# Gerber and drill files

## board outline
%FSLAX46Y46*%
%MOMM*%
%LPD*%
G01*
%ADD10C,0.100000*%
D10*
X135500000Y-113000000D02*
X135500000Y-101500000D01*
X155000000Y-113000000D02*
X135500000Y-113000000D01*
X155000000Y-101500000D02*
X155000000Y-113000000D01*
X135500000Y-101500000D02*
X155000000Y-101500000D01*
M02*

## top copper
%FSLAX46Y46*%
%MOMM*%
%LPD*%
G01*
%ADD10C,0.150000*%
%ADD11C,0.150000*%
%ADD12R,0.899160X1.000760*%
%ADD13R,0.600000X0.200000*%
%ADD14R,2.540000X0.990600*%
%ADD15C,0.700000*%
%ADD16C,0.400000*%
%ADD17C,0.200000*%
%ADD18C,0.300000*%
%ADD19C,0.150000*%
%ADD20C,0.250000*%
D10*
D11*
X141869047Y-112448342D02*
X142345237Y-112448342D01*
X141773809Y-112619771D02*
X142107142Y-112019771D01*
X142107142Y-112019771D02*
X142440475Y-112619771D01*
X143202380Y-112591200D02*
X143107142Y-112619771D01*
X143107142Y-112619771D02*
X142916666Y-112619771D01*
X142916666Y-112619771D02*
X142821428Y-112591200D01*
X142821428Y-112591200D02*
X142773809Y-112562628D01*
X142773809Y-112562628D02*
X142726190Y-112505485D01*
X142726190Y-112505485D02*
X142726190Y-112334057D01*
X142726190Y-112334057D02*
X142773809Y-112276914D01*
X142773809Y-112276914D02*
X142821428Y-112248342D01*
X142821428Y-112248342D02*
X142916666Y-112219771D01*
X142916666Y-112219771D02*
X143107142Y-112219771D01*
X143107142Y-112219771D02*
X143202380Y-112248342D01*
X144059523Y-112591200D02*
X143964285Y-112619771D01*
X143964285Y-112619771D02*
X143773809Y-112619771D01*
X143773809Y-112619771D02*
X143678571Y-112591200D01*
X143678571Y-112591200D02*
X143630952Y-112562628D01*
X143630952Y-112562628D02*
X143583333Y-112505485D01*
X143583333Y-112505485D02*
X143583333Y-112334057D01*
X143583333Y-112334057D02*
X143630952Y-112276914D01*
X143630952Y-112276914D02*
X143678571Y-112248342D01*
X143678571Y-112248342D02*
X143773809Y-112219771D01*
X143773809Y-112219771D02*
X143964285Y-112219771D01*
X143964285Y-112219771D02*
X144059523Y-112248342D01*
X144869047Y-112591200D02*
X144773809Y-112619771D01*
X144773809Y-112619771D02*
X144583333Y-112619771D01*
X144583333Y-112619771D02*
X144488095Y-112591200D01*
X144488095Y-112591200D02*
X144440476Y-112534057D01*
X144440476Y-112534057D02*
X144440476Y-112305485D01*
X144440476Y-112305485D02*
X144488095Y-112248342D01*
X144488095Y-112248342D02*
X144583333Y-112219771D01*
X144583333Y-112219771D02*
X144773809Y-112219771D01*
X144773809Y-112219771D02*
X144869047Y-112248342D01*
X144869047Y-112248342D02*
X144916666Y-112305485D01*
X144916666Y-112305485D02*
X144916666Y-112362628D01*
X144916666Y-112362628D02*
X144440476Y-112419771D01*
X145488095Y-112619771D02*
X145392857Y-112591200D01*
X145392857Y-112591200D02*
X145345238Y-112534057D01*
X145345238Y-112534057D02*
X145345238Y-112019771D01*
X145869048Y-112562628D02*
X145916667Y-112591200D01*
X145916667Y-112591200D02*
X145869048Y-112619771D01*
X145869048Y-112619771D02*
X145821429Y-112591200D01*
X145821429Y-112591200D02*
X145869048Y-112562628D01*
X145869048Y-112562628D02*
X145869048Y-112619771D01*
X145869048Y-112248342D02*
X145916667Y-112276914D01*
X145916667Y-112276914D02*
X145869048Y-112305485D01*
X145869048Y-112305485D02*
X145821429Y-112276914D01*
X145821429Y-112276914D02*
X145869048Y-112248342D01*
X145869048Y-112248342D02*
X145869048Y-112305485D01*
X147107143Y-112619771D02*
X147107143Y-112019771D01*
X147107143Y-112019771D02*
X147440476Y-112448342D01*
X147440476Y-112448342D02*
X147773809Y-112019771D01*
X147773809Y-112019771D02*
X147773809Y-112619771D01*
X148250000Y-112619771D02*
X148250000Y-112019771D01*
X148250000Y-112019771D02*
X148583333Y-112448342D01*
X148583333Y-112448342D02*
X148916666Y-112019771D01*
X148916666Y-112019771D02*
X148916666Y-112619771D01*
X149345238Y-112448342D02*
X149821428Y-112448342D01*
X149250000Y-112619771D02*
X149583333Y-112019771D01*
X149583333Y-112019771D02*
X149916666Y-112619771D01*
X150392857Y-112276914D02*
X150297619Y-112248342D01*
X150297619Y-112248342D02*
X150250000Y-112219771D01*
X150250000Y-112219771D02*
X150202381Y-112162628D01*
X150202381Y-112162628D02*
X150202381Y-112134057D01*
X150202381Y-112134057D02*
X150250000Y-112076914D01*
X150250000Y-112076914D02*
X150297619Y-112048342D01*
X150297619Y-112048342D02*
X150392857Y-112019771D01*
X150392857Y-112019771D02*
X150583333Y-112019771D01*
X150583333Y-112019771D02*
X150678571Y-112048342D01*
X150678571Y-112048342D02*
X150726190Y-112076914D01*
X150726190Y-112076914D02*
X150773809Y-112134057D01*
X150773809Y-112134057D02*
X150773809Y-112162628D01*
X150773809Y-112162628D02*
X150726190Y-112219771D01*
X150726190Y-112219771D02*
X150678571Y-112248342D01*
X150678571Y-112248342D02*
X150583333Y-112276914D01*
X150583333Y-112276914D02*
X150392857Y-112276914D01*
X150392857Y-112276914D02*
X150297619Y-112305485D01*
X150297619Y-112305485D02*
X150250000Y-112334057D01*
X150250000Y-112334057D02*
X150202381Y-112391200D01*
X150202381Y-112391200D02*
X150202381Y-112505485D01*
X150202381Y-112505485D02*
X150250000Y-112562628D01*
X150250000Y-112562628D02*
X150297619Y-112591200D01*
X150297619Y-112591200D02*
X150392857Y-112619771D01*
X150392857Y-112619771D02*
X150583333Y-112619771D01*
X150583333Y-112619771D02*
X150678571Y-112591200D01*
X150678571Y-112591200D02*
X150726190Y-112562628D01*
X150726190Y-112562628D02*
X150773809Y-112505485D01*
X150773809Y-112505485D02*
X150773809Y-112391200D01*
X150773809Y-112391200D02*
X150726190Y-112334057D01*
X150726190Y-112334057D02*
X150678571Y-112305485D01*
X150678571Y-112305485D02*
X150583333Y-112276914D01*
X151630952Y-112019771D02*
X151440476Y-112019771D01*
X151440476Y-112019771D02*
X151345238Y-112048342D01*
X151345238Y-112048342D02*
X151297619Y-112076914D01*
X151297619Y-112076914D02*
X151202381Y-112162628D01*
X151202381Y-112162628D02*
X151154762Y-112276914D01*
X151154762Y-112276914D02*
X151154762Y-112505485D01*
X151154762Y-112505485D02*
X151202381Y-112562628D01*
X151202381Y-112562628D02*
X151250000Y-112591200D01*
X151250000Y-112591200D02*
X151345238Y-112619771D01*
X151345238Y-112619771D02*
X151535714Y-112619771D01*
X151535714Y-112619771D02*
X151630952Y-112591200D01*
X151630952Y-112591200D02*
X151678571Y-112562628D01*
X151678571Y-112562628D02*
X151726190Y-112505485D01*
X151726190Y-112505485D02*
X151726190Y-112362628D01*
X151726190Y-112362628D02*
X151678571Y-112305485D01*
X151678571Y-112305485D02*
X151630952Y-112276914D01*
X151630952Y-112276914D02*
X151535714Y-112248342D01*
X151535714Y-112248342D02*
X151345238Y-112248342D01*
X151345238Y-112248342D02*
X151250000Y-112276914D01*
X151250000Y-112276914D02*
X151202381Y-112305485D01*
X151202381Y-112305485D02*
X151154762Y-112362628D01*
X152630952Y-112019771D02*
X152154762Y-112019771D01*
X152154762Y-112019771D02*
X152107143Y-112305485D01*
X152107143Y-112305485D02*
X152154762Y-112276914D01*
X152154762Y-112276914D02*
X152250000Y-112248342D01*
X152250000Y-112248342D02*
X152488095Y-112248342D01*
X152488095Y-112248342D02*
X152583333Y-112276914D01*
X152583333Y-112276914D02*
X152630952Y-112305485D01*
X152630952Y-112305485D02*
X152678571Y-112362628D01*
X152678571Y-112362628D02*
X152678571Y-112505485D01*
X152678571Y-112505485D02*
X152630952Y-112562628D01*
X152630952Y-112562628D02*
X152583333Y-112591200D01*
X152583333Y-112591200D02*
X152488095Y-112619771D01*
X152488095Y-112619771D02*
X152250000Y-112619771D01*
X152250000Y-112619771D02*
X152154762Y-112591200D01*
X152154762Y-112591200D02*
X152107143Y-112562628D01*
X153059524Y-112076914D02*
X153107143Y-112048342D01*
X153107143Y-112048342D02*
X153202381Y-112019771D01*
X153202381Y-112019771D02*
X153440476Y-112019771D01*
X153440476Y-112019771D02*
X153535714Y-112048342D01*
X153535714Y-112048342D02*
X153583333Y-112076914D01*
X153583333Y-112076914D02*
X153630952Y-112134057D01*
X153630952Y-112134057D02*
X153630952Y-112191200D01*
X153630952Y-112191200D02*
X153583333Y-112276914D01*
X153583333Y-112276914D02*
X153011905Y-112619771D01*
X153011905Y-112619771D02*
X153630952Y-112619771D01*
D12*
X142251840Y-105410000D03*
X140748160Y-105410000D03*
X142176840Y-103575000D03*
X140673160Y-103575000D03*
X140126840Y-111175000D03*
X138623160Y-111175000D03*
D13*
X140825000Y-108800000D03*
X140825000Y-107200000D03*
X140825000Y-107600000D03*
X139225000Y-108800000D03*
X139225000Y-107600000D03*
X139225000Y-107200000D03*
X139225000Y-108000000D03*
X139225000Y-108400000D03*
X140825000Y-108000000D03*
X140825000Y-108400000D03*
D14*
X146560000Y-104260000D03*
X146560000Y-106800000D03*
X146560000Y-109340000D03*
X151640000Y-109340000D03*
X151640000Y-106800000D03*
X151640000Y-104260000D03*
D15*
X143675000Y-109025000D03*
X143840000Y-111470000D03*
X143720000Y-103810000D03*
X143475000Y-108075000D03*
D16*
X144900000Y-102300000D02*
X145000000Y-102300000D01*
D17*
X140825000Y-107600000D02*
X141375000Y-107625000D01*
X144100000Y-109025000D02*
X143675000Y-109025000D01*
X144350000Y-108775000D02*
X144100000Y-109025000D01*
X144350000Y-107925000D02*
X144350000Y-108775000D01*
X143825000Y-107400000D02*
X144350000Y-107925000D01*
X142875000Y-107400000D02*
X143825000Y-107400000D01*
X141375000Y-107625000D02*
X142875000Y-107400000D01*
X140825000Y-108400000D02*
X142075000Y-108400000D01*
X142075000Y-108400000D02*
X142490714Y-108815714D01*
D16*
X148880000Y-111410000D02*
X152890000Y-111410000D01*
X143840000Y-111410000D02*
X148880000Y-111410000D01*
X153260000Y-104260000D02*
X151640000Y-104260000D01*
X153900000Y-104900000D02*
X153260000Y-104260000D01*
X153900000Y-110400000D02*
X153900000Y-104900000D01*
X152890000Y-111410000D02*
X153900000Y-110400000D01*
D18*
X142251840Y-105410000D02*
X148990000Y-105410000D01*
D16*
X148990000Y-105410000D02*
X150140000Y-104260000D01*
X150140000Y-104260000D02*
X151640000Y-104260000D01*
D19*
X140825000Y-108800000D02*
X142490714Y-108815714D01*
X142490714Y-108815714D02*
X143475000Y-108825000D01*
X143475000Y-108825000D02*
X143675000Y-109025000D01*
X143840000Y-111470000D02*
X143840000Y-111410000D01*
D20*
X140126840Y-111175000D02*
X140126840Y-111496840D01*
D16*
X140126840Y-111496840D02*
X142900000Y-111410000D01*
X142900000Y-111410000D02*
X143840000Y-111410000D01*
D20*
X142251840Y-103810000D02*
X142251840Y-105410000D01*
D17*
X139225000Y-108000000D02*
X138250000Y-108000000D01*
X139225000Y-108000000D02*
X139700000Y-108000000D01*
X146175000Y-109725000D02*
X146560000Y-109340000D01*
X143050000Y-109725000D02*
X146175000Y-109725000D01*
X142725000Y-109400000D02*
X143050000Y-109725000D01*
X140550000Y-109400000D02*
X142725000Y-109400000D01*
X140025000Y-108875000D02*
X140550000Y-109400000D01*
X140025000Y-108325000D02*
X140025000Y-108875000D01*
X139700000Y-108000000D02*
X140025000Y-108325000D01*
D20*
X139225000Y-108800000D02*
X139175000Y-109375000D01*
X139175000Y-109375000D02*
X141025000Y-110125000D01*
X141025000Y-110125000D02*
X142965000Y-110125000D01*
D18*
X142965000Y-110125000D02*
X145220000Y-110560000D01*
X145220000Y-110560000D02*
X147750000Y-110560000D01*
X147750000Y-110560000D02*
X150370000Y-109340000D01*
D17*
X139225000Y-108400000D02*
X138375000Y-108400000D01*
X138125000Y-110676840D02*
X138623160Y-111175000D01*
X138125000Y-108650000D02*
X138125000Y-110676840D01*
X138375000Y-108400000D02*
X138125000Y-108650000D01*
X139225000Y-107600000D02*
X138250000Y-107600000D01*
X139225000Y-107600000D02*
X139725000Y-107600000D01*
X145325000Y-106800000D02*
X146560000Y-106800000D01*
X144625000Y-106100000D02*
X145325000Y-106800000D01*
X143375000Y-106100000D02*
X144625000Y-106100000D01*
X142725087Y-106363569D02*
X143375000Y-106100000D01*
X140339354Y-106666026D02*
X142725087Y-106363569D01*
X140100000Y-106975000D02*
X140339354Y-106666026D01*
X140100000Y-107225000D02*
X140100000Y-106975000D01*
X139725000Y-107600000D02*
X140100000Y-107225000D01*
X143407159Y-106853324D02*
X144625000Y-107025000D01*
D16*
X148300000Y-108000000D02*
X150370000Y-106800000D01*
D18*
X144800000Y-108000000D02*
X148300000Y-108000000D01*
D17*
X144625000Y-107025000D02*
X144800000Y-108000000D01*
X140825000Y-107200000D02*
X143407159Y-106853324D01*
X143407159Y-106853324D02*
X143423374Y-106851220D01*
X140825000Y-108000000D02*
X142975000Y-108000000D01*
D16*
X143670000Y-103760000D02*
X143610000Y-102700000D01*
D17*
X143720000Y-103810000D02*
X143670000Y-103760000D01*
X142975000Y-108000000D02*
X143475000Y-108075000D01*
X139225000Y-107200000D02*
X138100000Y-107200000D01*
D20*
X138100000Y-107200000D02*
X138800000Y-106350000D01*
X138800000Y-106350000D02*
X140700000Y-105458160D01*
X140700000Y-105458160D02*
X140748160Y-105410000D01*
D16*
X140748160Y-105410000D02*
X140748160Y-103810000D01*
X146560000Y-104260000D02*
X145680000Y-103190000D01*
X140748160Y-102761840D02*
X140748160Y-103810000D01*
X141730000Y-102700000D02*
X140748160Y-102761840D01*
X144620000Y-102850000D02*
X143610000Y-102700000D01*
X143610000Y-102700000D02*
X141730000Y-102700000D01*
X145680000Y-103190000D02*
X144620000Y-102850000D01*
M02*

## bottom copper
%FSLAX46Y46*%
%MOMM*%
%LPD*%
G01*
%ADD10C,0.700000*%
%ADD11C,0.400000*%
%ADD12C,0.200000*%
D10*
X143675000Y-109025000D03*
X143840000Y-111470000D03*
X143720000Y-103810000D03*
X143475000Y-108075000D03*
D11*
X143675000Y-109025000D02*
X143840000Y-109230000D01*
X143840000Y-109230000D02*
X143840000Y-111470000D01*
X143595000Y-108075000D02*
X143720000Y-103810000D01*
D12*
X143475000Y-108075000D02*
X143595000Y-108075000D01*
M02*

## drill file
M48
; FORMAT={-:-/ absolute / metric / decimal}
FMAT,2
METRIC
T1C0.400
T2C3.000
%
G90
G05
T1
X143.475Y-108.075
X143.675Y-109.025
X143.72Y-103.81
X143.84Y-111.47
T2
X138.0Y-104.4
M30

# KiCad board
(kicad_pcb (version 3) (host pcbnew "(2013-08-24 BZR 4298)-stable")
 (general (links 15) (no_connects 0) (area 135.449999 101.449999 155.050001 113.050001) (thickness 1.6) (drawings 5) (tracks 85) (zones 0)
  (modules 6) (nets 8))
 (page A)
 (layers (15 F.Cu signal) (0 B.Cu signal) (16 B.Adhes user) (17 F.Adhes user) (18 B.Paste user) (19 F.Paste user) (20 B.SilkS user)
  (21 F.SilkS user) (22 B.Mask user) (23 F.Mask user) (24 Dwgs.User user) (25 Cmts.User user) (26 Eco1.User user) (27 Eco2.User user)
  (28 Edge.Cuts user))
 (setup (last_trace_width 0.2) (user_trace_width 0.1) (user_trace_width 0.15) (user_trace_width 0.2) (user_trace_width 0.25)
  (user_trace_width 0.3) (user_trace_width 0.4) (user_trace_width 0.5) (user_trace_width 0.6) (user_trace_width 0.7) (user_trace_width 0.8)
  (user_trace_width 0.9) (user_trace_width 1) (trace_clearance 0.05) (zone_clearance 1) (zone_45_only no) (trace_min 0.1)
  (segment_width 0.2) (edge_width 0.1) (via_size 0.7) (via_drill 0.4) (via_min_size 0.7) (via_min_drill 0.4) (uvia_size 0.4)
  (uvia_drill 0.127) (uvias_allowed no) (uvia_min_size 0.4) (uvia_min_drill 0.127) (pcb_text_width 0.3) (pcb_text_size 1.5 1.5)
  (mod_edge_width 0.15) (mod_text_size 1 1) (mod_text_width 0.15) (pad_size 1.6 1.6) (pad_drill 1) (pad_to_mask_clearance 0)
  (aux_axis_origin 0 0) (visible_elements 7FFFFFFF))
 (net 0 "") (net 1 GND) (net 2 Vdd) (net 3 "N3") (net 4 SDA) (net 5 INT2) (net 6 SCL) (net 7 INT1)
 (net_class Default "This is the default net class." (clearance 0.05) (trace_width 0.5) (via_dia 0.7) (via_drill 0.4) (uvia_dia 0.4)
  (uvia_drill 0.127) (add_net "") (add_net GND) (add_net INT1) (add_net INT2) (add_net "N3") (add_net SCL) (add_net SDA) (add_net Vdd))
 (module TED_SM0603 (layer F.Cu) (at 141.5 105.41)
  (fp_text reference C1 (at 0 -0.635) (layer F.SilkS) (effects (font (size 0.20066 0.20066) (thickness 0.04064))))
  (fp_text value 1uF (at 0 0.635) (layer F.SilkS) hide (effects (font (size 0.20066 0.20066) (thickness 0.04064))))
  (pad 2 smd rect (at 0.75184 0) (size 0.89916 1.00076) (layers F.Cu F.Paste F.Mask) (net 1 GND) (clearance 0.1))
  (pad 1 smd rect (at -0.75184 0) (size 0.89916 1.00076) (layers F.Cu F.Paste F.Mask) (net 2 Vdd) (clearance 0.1)))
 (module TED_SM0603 (layer F.Cu) (at 141.425 103.575)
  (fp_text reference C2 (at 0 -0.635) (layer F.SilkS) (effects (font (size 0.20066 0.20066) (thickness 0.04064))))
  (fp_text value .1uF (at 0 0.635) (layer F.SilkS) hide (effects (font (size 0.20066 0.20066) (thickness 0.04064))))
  (pad 2 smd rect (at 0.75184 0) (size 0.89916 1.00076) (layers F.Cu F.Paste F.Mask) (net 1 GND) (clearance 0.1))
  (pad 1 smd rect (at -0.75184 0) (size 0.89916 1.00076) (layers F.Cu F.Paste F.Mask) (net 2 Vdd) (clearance 0.1)))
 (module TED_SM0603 (layer F.Cu) (at 139.375 111.175)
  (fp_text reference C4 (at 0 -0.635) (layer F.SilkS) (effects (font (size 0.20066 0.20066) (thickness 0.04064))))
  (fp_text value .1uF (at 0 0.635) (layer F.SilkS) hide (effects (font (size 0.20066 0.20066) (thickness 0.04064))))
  (pad 2 smd rect (at 0.75184 0) (size 0.89916 1.00076) (layers F.Cu F.Paste F.Mask) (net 1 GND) (clearance 0.1))
  (pad 1 smd rect (at -0.75184 0) (size 0.89916 1.00076) (layers F.Cu F.Paste F.Mask) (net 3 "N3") (clearance 0.1)))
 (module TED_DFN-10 (layer F.Cu) (at 140.025 108)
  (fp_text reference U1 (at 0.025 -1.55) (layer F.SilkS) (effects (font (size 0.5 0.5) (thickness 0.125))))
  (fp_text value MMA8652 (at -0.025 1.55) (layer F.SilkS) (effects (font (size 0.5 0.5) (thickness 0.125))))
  (pad 6 smd rect (at 0.8 0.8 270) (size 0.2 0.6) (layers F.Cu F.Paste F.Mask) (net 1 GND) (clearance 0.1))
  (pad 10 smd rect (at 0.8 -0.8 270) (size 0.2 0.6) (layers F.Cu F.Paste F.Mask) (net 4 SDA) (clearance 0.1))
  (pad 9 smd rect (at 0.8 -0.4 270) (size 0.2 0.6) (layers F.Cu F.Paste F.Mask) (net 1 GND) (clearance 0.1))
  (pad 5 smd rect (at -0.8 0.8 270) (size 0.2 0.6) (layers F.Cu F.Paste F.Mask) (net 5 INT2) (clearance 0.1))
  (pad 2 smd rect (at -0.8 -0.4 270) (size 0.2 0.6) (layers F.Cu F.Paste F.Mask) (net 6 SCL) (clearance 0.1))
  (pad 1 smd rect (at -0.8 -0.8 270) (size 0.2 0.6) (layers F.Cu F.Paste F.Mask) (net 2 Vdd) (clearance 0.1))
  (pad 3 smd rect (at -0.8 0 270) (size 0.2 0.6) (layers F.Cu F.Paste F.Mask) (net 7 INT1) (clearance 0.1))
  (pad 4 smd rect (at -0.8 0.4 270) (size 0.2 0.6) (layers F.Cu F.Paste F.Mask) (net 3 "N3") (clearance 0.1))
  (pad 8 smd rect (at 0.8 0 270) (size 0.2 0.6) (layers F.Cu F.Paste F.Mask) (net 2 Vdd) (clearance 0.1))
  (pad 7 smd rect (at 0.8 0.4 270) (size 0.2 0.6) (layers F.Cu F.Paste F.Mask) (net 1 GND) (clearance 0.1)))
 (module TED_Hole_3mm (layer F.Cu) (at 138 104.4)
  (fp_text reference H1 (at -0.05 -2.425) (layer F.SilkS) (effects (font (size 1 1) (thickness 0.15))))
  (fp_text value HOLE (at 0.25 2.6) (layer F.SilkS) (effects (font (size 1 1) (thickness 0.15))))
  (pad "" np_thru_hole circle (at 0 0) (size 3 3) (drill 3) (layers *.Cu *.Mask F.SilkS)))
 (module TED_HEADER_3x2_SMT (layer F.Cu) (at 149.1 106.8 270)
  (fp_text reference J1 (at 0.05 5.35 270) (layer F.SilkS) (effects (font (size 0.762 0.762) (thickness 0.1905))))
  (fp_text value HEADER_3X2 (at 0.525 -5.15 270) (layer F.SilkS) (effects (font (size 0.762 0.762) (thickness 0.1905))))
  (pad 1 smd rect (at -2.54 2.54 270) (size 0.9906 2.54) (layers F.Cu F.Paste F.Mask) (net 2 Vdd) (clearance 0.3))
  (pad 2 smd rect (at 0 2.54 270) (size 0.9906 2.54) (layers F.Cu F.Paste F.Mask) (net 6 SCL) (clearance 0.3))
  (pad 3 smd rect (at 2.54 2.54 270) (size 0.9906 2.54) (layers F.Cu F.Paste F.Mask) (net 7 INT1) (clearance 0.3))
  (pad 4 smd rect (at 2.54 -2.54 270) (size 0.9906 2.54) (layers F.Cu F.Paste F.Mask) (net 5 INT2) (clearance 0.3))
  (pad 5 smd rect (at 0 -2.54 270) (size 0.9906 2.54) (layers F.Cu F.Paste F.Mask) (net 4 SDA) (clearance 0.3))
  (pad 6 smd rect (at -2.54 -2.54 270) (size 0.9906 2.54) (layers F.Cu F.Paste F.Mask) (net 1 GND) (clearance 0.3)))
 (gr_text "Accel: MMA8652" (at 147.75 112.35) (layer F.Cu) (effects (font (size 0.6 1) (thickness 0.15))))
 (gr_line (start 135.5 113) (end 135.5 101.5) (angle 90) (layer Edge.Cuts) (width 0.1))
 (gr_line (start 155 113) (end 135.5 113) (angle 90) (layer Edge.Cuts) (width 0.1))
 (gr_line (start 155 101.5) (end 155 113) (angle 90) (layer Edge.Cuts) (width 0.1))
 (gr_line (start 135.5 101.5) (end 155 101.5) (angle 90) (layer Edge.Cuts) (width 0.1))
 (segment (start 144.9 102.3) (end 145 102.3) (width 0.4) (layer F.Cu) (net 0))
 (segment (start 140.825 107.6) (end 141.375 107.625) (width 0.2) (layer F.Cu) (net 1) (status 400000))
 (segment (start 144.1 109.025) (end 143.675 109.025) (width 0.2) (layer F.Cu) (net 1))
 (segment (start 144.35 108.775) (end 144.1 109.025) (width 0.2) (layer F.Cu) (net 1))
 (segment (start 144.35 107.925) (end 144.35 108.775) (width 0.2) (layer F.Cu) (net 1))
 (segment (start 143.825 107.4) (end 144.35 107.925) (width 0.2) (layer F.Cu) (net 1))
 (segment (start 142.875 107.4) (end 143.825 107.4) (width 0.2) (layer F.Cu) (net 1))
 (segment (start 141.375 107.625) (end 142.875 107.4) (width 0.2) (layer F.Cu) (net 1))
 (segment (start 140.825 108.4) (end 142.075 108.4) (width 0.2) (layer F.Cu) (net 1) (status 400000))
 (segment (start 142.075 108.4) (end 142.490714 108.815714) (width 0.2) (layer F.Cu) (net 1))
 (segment (start 148.88 111.41) (end 152.89 111.41) (width 0.4) (layer F.Cu) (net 1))
 (segment (start 143.84 111.41) (end 148.88 111.41) (width 0.4) (layer F.Cu) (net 1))
 (segment (start 153.26 104.26) (end 151.64 104.26) (width 0.4) (layer F.Cu) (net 1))
 (segment (start 153.9 104.9) (end 153.26 104.26) (width 0.4) (layer F.Cu) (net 1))
 (segment (start 153.9 110.4) (end 153.9 104.9) (width 0.4) (layer F.Cu) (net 1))
 (segment (start 152.89 111.41) (end 153.9 110.4) (width 0.4) (layer F.Cu) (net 1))
 (segment (start 142.25184 105.41) (end 148.99 105.41) (width 0.3) (layer F.Cu) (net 1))
 (segment (start 148.99 105.41) (end 150.14 104.26) (width 0.4) (layer F.Cu) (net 1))
 (segment (start 150.14 104.26) (end 151.64 104.26) (width 0.4) (layer F.Cu) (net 1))
 (segment (start 140.825 108.8) (end 142.490714 108.815714) (width 0.15) (layer F.Cu) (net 1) (status 400010))
 (segment (start 142.490714 108.815714) (end 143.475 108.825) (width 0.15) (layer F.Cu) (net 1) (status 10))
 (segment (start 143.475 108.825) (end 143.675 109.025) (width 0.15) (layer F.Cu) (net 1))
 (via (at 143.675 109.025) (size 0.7) (layers F.Cu B.Cu) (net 1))
 (segment (start 143.675 109.025) (end 143.84 109.23) (width 0.4) (layer B.Cu) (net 1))
 (segment (start 143.84 109.23) (end 143.84 111.47) (width 0.4) (layer B.Cu) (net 1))
 (via (at 143.84 111.47) (size 0.7) (layers F.Cu B.Cu) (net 1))
 (segment (start 143.84 111.47) (end 143.84 111.41) (width 0.15) (layer F.Cu) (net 1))
 (segment (start 140.12684 111.175) (end 140.12684 111.49684) (width 0.25) (layer F.Cu) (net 1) (status 30))
 (segment (start 140.12684 111.49684) (end 142.9 111.41) (width 0.4) (layer F.Cu) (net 1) (status 10))
 (segment (start 142.9 111.41) (end 143.84 111.41) (width 0.4) (layer F.Cu) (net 1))
 (segment (start 142.25184 103.81) (end 142.25184 105.41) (width 0.25) (layer F.Cu) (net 1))
 (segment (start 139.225 108) (end 138.25 108) (width 0.2) (layer F.Cu) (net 7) (status 400000))
 (segment (start 139.225 108) (end 139.7 108) (width 0.2) (layer F.Cu) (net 7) (status 400000))
 (segment (start 146.175 109.725) (end 146.56 109.34) (width 0.2) (layer F.Cu) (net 7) (status C00000))
 (segment (start 143.05 109.725) (end 146.175 109.725) (width 0.2) (layer F.Cu) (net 7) (status 800000))
 (segment (start 142.725 109.4) (end 143.05 109.725) (width 0.2) (layer F.Cu) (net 7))
 (segment (start 140.55 109.4) (end 142.725 109.4) (width 0.2) (layer F.Cu) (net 7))
 (segment (start 140.025 108.875) (end 140.55 109.4) (width 0.2) (layer F.Cu) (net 7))
 (segment (start 140.025 108.325) (end 140.025 108.875) (width 0.2) (layer F.Cu) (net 7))
 (segment (start 139.7 108) (end 140.025 108.325) (width 0.2) (layer F.Cu) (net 7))
 (segment (start 139.225 108.8) (end 139.175 109.375) (width 0.25) (layer F.Cu) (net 5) (status 400010))
 (segment (start 139.175 109.375) (end 141.025 110.125) (width 0.25) (layer F.Cu) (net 5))
 (segment (start 141.025 110.125) (end 142.965 110.125) (width 0.25) (layer F.Cu) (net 5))
 (segment (start 142.965 110.125) (end 145.22 110.56) (width 0.3) (layer F.Cu) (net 5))
 (segment (start 145.22 110.56) (end 147.75 110.56) (width 0.3) (layer F.Cu) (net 5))
 (segment (start 147.75 110.56) (end 150.37 109.34) (width 0.3) (layer F.Cu) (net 5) (status 20))
 (segment (start 139.225 108.4) (end 138.375 108.4) (width 0.2) (layer F.Cu) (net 3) (status 400000))
 (segment (start 138.125 110.67684) (end 138.62316 111.175) (width 0.2) (layer F.Cu) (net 3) (status 800000))
 (segment (start 138.125 108.65) (end 138.125 110.67684) (width 0.2) (layer F.Cu) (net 3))
 (segment (start 138.375 108.4) (end 138.125 108.65) (width 0.2) (layer F.Cu) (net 3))
 (segment (start 139.225 107.6) (end 138.25 107.6) (width 0.2) (layer F.Cu) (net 6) (status 400000))
 (segment (start 139.225 107.6) (end 139.725 107.6) (width 0.2) (layer F.Cu) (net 6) (status 400000))
 (segment (start 145.325 106.8) (end 146.56 106.8) (width 0.2) (layer F.Cu) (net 6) (status C00000))
 (segment (start 144.625 106.1) (end 145.325 106.8) (width 0.2) (layer F.Cu) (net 6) (status 800000))
 (segment (start 143.375 106.1) (end 144.625 106.1) (width 0.2) (layer F.Cu) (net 6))
 (segment (start 142.725087 106.363569) (end 143.375 106.1) (width 0.2) (layer F.Cu) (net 6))
 (segment (start 140.339354 106.666026) (end 142.725087 106.363569) (width 0.2) (layer F.Cu) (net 6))
 (segment (start 140.1 106.975) (end 140.339354 106.666026) (width 0.2) (layer F.Cu) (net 6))
 (segment (start 140.1 107.225) (end 140.1 106.975) (width 0.2) (layer F.Cu) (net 6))
 (segment (start 139.725 107.6) (end 140.1 107.225) (width 0.2) (layer F.Cu) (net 6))
 (segment (start 143.407159 106.853324) (end 144.625 107.025) (width 0.2) (layer F.Cu) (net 4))
 (segment (start 148.3 108) (end 150.37 106.8) (width 0.4) (layer F.Cu) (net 4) (status 20))
 (segment (start 144.8 108) (end 148.3 108) (width 0.3) (layer F.Cu) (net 4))
 (segment (start 144.625 107.025) (end 144.8 108) (width 0.2) (layer F.Cu) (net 4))
 (segment (start 140.825 107.2) (end 143.407159 106.853324) (width 0.2) (layer F.Cu) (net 4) (status 400010))
 (segment (start 143.407159 106.853324) (end 143.423374 106.85122) (width 0.2) (layer F.Cu) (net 4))
 (segment (start 140.825 108) (end 142.975 108) (width 0.2) (layer F.Cu) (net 2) (status 400010))
 (segment (start 143.67 103.76) (end 143.61 102.7) (width 0.4) (layer F.Cu) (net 2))
 (segment (start 143.72 103.81) (end 143.67 103.76) (width 0.2) (layer F.Cu) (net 2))
 (via (at 143.72 103.81) (size 0.7) (layers F.Cu B.Cu) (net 2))
 (segment (start 143.595 108.075) (end 143.72 103.81) (width 0.4) (layer B.Cu) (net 2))
 (segment (start 143.475 108.075) (end 143.595 108.075) (width 0.2) (layer B.Cu) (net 2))
 (via (at 143.475 108.075) (size 0.7) (layers F.Cu B.Cu) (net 2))
 (segment (start 142.975 108) (end 143.475 108.075) (width 0.2) (layer F.Cu) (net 2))
 (segment (start 139.225 107.2) (end 138.1 107.2) (width 0.2) (layer F.Cu) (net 2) (status 400010))
 (segment (start 138.1 107.2) (end 138.8 106.35) (width 0.25) (layer F.Cu) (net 2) (status 10))
 (segment (start 138.8 106.35) (end 140.7 105.45816) (width 0.25) (layer F.Cu) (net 2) (status 10))
 (segment (start 140.7 105.45816) (end 140.74816 105.41) (width 0.25) (layer F.Cu) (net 2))
 (segment (start 140.74816 105.41) (end 140.74816 103.81) (width 0.4) (layer F.Cu) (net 2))
 (segment (start 146.56 104.26) (end 145.68 103.19) (width 0.4) (layer F.Cu) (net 2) (status 10))
 (segment (start 140.74816 102.76184) (end 140.74816 103.81) (width 0.4) (layer F.Cu) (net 2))
 (segment (start 141.73 102.7) (end 140.74816 102.76184) (width 0.4) (layer F.Cu) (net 2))
 (segment (start 144.62 102.85) (end 143.61 102.7) (width 0.4) (layer F.Cu) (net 2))
 (segment (start 143.61 102.7) (end 141.73 102.7) (width 0.4) (layer F.Cu) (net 2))
 (segment (start 145.68 103.19) (end 144.62 102.85) (width 0.4) (layer F.Cu) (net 2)))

